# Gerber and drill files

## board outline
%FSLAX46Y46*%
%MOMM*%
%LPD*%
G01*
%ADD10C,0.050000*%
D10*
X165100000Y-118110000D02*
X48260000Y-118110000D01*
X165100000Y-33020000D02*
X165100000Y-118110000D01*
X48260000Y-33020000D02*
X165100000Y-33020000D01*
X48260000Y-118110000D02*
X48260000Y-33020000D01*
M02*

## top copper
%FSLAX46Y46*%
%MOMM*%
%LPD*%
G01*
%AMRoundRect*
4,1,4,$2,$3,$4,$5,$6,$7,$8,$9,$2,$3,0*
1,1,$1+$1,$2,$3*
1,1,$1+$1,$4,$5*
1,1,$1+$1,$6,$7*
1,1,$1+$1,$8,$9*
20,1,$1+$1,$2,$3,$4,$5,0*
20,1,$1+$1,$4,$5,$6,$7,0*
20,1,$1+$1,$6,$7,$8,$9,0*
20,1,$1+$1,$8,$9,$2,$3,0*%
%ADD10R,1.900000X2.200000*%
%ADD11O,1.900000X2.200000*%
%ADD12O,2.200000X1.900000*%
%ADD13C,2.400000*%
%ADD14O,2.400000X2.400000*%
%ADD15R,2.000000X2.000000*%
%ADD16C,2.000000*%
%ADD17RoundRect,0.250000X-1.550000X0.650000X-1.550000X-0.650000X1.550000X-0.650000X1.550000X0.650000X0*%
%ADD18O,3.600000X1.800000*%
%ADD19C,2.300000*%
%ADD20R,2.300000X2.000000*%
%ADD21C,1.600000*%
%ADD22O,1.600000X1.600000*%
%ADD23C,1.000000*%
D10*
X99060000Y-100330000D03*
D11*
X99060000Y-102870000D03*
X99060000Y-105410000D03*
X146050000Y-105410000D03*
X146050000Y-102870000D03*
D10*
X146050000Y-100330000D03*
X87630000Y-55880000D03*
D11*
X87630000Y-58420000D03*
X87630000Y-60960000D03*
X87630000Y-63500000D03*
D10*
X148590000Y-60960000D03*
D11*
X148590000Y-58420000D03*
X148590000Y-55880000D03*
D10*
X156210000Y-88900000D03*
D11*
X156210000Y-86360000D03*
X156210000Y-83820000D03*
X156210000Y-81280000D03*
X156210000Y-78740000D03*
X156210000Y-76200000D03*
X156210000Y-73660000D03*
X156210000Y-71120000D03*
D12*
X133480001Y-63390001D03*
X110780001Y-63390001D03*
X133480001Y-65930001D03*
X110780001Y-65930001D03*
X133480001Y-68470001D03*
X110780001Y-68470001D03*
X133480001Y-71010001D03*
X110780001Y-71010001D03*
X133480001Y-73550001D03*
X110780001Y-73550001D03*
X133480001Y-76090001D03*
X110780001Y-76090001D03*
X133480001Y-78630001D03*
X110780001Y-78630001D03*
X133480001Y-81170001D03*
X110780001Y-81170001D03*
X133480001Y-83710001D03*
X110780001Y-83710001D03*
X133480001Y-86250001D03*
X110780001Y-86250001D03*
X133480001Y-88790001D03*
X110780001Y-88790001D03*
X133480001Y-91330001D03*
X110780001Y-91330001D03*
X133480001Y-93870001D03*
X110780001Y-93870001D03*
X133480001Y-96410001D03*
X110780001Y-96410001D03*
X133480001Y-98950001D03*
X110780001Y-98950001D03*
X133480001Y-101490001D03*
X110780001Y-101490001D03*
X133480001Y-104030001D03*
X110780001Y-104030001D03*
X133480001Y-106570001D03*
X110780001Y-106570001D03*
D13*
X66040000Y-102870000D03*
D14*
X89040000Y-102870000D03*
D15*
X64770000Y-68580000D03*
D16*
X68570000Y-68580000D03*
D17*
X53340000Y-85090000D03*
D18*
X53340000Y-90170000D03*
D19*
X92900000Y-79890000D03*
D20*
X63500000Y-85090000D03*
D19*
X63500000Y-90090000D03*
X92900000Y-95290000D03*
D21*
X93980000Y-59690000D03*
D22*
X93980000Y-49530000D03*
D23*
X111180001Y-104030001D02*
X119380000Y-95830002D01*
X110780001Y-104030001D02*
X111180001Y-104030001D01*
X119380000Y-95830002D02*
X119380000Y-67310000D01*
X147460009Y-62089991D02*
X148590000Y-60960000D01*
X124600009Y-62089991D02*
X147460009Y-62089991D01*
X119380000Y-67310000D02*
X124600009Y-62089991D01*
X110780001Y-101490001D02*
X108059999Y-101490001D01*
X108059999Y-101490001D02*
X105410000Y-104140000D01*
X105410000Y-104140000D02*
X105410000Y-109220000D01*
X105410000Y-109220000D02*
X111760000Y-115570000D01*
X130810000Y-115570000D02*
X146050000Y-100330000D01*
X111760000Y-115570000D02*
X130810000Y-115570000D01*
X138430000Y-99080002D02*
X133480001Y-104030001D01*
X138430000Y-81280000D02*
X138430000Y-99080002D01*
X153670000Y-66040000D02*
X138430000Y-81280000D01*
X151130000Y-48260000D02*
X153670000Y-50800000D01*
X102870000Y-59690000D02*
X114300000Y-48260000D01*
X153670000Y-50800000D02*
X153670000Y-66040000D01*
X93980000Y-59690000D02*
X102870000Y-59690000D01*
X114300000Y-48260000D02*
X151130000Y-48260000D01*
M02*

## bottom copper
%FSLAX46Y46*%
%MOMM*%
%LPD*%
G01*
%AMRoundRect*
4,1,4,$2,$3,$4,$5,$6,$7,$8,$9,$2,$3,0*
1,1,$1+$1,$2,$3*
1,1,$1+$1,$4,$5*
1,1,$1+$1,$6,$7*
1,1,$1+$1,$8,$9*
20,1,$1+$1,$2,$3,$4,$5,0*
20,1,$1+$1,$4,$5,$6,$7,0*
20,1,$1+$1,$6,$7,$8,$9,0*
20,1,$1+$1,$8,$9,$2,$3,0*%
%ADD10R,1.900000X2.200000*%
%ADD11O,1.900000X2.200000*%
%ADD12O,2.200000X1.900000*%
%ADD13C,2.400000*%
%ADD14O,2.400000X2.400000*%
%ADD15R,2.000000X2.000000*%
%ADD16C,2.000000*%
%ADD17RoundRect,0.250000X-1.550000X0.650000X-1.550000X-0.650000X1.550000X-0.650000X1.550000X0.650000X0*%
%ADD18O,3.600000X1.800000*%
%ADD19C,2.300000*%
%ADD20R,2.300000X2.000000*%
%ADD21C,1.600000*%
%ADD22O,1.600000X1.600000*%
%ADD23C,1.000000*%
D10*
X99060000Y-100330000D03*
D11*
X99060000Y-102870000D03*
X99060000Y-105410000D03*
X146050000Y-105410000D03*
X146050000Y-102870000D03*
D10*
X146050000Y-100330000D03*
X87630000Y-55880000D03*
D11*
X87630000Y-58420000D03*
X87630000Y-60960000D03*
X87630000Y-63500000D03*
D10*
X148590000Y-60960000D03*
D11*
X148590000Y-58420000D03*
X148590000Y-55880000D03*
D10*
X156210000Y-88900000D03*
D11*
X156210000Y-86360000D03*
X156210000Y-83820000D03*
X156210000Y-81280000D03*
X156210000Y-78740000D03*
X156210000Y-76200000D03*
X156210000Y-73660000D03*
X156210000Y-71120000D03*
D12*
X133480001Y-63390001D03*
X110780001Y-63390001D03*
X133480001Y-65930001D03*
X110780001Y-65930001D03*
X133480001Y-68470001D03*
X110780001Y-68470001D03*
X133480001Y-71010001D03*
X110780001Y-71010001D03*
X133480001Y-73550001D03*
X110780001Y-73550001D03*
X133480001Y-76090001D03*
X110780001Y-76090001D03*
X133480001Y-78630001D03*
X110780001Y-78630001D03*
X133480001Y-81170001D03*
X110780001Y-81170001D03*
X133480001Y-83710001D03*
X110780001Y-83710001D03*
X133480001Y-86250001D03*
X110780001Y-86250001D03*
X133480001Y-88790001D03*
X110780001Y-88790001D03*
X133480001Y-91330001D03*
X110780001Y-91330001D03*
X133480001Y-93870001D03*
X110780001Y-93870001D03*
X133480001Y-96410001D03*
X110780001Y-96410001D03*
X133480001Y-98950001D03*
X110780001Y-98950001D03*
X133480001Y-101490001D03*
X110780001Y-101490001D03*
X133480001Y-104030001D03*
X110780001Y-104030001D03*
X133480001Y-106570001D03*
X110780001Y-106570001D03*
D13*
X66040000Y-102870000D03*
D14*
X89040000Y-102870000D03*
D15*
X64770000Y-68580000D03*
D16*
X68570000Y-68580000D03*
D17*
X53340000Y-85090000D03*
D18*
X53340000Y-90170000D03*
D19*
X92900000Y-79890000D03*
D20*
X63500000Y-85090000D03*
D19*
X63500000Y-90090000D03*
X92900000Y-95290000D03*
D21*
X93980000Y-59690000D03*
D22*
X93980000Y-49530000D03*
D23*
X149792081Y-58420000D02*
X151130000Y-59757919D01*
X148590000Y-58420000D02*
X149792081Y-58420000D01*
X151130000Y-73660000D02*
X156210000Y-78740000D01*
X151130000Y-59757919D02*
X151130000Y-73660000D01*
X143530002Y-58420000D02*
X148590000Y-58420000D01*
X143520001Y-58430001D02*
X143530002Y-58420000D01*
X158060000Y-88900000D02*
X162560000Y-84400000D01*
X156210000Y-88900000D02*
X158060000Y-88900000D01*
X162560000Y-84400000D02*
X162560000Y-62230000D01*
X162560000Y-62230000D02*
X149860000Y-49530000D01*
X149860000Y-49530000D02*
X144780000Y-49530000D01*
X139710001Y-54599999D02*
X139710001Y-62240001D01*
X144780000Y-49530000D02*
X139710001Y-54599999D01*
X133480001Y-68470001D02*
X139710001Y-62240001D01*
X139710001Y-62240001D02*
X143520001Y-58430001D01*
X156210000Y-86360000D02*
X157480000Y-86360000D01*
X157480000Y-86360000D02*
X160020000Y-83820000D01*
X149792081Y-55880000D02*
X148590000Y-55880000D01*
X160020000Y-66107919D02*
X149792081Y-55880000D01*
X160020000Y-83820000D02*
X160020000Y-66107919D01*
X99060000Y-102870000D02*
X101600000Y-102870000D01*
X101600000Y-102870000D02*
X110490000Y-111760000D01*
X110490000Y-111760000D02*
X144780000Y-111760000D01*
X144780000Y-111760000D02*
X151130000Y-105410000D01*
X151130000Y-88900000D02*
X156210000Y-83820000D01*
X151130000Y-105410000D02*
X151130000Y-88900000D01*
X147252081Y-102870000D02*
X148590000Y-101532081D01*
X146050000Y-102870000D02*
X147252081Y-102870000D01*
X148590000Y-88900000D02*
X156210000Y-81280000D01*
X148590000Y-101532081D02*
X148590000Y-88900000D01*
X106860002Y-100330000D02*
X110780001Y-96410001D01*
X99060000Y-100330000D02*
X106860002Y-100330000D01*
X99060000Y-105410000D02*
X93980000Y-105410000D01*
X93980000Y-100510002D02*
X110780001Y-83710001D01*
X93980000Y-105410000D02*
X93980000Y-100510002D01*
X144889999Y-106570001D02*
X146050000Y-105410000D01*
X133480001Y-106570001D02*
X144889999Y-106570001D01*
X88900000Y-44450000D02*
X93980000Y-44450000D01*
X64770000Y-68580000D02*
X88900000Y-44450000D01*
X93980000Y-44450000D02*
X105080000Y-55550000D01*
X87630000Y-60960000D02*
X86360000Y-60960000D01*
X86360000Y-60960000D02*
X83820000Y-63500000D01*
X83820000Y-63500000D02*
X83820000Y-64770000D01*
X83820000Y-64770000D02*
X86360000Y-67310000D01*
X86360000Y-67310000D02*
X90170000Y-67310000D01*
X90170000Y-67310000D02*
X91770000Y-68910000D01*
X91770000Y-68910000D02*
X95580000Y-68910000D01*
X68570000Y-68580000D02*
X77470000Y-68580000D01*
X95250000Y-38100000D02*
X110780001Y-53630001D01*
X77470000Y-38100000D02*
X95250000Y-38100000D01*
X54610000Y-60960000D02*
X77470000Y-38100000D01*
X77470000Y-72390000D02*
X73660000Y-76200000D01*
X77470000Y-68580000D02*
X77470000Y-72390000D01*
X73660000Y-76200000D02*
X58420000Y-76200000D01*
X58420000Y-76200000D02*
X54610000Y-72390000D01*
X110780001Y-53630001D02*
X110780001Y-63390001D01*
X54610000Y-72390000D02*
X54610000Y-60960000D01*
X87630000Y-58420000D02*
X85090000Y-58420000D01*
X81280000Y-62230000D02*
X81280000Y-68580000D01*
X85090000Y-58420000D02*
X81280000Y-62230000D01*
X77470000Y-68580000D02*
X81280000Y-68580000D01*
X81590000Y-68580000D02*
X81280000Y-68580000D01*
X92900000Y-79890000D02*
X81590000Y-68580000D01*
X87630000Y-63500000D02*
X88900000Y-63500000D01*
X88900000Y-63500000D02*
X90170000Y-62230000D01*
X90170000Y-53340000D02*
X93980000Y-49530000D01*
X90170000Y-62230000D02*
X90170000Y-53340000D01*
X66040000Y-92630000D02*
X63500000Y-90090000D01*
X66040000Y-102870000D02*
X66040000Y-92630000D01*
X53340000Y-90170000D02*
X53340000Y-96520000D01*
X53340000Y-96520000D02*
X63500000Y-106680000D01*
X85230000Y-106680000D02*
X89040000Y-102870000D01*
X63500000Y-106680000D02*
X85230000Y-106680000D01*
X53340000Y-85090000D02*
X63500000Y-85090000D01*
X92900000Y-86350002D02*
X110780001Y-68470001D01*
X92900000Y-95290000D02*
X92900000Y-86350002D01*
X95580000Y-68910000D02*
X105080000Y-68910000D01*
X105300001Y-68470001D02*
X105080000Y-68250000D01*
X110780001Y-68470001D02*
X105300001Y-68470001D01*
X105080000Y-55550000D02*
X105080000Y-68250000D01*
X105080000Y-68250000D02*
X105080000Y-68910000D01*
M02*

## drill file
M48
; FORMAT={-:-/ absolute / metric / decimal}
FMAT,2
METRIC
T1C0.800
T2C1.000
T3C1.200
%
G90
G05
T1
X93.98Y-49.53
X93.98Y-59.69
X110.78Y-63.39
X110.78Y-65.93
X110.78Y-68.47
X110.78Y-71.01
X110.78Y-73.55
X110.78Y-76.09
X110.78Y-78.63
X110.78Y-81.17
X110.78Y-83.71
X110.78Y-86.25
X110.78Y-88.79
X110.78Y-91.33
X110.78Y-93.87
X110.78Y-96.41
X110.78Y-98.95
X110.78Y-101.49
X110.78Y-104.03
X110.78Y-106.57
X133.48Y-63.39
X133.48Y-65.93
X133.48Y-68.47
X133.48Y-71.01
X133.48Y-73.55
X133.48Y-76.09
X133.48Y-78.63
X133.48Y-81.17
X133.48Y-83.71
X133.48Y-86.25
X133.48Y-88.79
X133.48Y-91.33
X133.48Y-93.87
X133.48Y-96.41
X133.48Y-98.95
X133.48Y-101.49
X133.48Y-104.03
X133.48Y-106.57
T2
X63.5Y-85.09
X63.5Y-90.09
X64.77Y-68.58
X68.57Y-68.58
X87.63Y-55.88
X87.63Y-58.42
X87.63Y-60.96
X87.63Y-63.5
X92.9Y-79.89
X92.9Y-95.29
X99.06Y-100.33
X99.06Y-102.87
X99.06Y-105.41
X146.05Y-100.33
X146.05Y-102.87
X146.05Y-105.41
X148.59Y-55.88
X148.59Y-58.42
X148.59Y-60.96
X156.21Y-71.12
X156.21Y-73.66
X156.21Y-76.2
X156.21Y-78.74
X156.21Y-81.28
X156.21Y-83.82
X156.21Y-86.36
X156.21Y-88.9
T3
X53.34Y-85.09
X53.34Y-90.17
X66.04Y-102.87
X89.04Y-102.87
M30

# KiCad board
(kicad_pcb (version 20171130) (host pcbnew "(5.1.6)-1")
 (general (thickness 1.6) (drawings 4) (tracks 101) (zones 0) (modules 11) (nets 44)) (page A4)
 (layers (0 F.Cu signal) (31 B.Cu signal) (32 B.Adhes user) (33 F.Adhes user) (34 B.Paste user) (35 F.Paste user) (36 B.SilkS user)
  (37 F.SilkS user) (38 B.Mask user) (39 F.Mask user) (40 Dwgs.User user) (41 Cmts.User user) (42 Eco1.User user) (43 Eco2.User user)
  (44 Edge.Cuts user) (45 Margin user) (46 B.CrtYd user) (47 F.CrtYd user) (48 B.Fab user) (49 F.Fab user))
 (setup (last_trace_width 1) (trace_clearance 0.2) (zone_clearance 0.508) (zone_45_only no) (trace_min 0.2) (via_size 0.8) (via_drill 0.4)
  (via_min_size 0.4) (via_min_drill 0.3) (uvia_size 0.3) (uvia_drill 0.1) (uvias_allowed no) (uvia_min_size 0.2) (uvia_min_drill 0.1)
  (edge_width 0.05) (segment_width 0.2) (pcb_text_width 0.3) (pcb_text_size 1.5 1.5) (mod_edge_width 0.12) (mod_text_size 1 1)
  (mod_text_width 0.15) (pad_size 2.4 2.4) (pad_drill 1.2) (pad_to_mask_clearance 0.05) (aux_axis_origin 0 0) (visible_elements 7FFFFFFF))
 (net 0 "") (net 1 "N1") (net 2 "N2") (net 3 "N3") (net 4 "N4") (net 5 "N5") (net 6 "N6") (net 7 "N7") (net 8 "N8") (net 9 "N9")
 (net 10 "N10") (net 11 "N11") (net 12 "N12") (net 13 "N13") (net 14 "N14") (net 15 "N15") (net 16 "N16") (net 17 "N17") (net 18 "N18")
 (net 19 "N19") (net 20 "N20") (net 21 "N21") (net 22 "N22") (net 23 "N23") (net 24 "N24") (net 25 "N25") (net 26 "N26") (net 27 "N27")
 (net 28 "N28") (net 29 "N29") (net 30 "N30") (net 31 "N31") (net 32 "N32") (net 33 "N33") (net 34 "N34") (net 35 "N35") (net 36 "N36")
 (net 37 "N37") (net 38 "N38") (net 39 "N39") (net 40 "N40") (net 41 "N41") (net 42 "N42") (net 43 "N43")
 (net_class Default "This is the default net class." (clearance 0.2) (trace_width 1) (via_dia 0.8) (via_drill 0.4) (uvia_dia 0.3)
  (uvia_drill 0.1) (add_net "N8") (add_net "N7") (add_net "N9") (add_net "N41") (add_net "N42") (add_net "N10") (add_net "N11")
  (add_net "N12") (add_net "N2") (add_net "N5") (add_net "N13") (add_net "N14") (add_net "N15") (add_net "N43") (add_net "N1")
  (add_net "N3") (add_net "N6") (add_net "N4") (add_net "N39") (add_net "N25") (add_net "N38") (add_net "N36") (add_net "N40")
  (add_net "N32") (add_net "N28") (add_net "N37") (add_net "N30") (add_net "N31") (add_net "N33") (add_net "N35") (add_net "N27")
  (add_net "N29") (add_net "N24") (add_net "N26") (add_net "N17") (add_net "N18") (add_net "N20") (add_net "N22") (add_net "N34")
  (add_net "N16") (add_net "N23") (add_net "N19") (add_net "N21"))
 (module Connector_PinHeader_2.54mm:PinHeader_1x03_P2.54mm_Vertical (layer F.Cu) (at 99.06 100.33)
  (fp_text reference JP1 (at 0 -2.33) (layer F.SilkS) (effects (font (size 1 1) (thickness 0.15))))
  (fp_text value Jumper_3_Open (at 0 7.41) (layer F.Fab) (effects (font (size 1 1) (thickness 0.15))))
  (pad 1 thru_hole rect (at 0 0) (size 1.9 2.2) (drill 1) (layers *.Cu *.Mask) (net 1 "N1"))
  (pad 2 thru_hole oval (at 0 2.54) (size 1.9 2.2) (drill 1) (layers *.Cu *.Mask) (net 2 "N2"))
  (pad 3 thru_hole oval (at 0 5.08) (size 1.9 2.2) (drill 1) (layers *.Cu *.Mask) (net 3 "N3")))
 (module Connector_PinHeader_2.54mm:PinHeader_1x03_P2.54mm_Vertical (layer F.Cu) (at 146.05 100.33)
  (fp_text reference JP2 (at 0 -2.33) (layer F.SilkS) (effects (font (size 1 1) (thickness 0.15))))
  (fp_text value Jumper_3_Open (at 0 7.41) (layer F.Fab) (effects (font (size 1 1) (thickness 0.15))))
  (pad 3 thru_hole oval (at 0 5.08) (size 1.9 2.2) (drill 1) (layers *.Cu *.Mask) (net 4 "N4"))
  (pad 2 thru_hole oval (at 0 2.54) (size 1.9 2.2) (drill 1) (layers *.Cu *.Mask) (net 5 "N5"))
  (pad 1 thru_hole rect (at 0 0) (size 1.9 2.2) (drill 1) (layers *.Cu *.Mask) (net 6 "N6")))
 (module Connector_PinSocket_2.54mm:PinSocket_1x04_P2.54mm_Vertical (layer F.Cu) (at 87.63 55.88)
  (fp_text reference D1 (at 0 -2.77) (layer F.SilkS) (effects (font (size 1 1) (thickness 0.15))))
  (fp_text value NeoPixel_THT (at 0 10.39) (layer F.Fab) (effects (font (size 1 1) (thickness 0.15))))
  (pad 1 thru_hole rect (at 0 0) (size 1.9 2.2) (drill 1) (layers *.Cu *.Mask) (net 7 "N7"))
  (pad 2 thru_hole oval (at 0 2.54) (size 1.9 2.2) (drill 1) (layers *.Cu *.Mask) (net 7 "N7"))
  (pad 3 thru_hole oval (at 0 5.08) (size 1.9 2.2) (drill 1) (layers *.Cu *.Mask) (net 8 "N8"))
  (pad 4 thru_hole oval (at 0 7.62) (size 1.9 2.2) (drill 1) (layers *.Cu *.Mask) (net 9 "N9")))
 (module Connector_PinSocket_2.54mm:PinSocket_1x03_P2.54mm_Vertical (layer F.Cu) (at 148.59 60.96 180)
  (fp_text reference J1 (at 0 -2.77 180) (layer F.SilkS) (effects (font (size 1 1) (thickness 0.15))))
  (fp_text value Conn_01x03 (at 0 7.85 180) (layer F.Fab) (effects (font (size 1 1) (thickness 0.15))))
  (pad 1 thru_hole rect (at 0 0 180) (size 1.9 2.2) (drill 1) (layers *.Cu *.Mask) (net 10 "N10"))
  (pad 2 thru_hole oval (at 0 2.54 180) (size 1.9 2.2) (drill 1) (layers *.Cu *.Mask) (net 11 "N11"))
  (pad 3 thru_hole oval (at 0 5.08 180) (size 1.9 2.2) (drill 1) (layers *.Cu *.Mask) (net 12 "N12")))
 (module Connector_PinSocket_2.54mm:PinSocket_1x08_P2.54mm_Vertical (layer F.Cu) (at 156.21 88.9 180)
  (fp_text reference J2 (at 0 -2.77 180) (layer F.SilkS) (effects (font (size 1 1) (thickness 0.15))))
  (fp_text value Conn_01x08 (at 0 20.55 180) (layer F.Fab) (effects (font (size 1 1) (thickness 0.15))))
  (pad 1 thru_hole rect (at 0 0 180) (size 1.9 2.2) (drill 1) (layers *.Cu *.Mask) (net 11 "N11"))
  (pad 2 thru_hole oval (at 0 2.54 180) (size 1.9 2.2) (drill 1) (layers *.Cu *.Mask) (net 12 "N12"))
  (pad 3 thru_hole oval (at 0 5.08 180) (size 1.9 2.2) (drill 1) (layers *.Cu *.Mask) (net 2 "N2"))
  (pad 4 thru_hole oval (at 0 7.62 180) (size 1.9 2.2) (drill 1) (layers *.Cu *.Mask) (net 5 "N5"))
  (pad 5 thru_hole oval (at 0 10.16 180) (size 1.9 2.2) (drill 1) (layers *.Cu *.Mask) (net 11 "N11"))
  (pad 6 thru_hole oval (at 0 12.7 180) (size 1.9 2.2) (drill 1) (layers *.Cu *.Mask) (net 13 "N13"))
  (pad 7 thru_hole oval (at 0 15.24 180) (size 1.9 2.2) (drill 1) (layers *.Cu *.Mask) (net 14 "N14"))
  (pad 8 thru_hole oval (at 0 17.78 180) (size 1.9 2.2) (drill 1) (layers *.Cu *.Mask) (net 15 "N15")))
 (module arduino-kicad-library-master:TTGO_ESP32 (layer F.Cu) (at 122.130001 86.250001)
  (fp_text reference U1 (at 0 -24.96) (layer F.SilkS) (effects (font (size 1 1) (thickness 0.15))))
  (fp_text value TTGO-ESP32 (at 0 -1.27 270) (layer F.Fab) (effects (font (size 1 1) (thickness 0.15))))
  (pad GND thru_hole oval (at 11.35 -22.86 270) (size 1.9 2.2) (drill 0.8) (layers *.Cu *.Mask) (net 7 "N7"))
  (pad GND thru_hole oval (at -11.35 -22.86 270) (size 1.9 2.2) (drill 0.8) (layers *.Cu *.Mask) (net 7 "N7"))
  (pad 5V thru_hole oval (at 11.35 -20.32 270) (size 1.9 2.2) (drill 0.8) (layers *.Cu *.Mask) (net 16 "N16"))
  (pad 5V thru_hole oval (at -11.35 -20.32 270) (size 1.9 2.2) (drill 0.8) (layers *.Cu *.Mask) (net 16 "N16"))
  (pad 3V3 thru_hole oval (at 11.35 -17.78 270) (size 1.9 2.2) (drill 0.8) (layers *.Cu *.Mask) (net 8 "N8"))
  (pad 3V3 thru_hole oval (at -11.35 -17.78 270) (size 1.9 2.2) (drill 0.8) (layers *.Cu *.Mask) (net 8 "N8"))
  (pad 36 thru_hole oval (at 11.35 -15.24 270) (size 1.9 2.2) (drill 0.8) (layers *.Cu *.Mask) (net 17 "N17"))
  (pad GND thru_hole oval (at -11.35 -15.24 270) (size 1.9 2.2) (drill 0.8) (layers *.Cu *.Mask) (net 7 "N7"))
  (pad 37 thru_hole oval (at 11.35 -12.7 270) (size 1.9 2.2) (drill 0.8) (layers *.Cu *.Mask) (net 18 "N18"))
  (pad RX thru_hole oval (at -11.35 -12.7 270) (size 1.9 2.2) (drill 0.8) (layers *.Cu *.Mask) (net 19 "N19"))
  (pad 38 thru_hole oval (at 11.35 -10.16 270) (size 1.9 2.2) (drill 0.8) (layers *.Cu *.Mask) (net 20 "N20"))
  (pad TX thru_hole oval (at -11.35 -10.16 270) (size 1.9 2.2) (drill 0.8) (layers *.Cu *.Mask) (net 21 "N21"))
  (pad 39 thru_hole oval (at 11.35 -7.62 270) (size 1.9 2.2) (drill 0.8) (layers *.Cu *.Mask) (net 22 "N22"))
  (pad RST thru_hole oval (at -11.35 -7.62 270) (size 1.9 2.2) (drill 0.8) (layers *.Cu *.Mask) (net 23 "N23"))
  (pad 34 thru_hole oval (at 11.35 -5.08 270) (size 1.9 2.2) (drill 0.8) (layers *.Cu *.Mask) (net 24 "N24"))
  (pad 0 thru_hole oval (at -11.35 -5.08 270) (size 1.9 2.2) (drill 0.8) (layers *.Cu *.Mask) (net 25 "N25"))
  (pad 35 thru_hole oval (at 11.35 -2.54 270) (size 1.9 2.2) (drill 0.8) (layers *.Cu *.Mask) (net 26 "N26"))
  (pad 22 thru_hole oval (at -11.35 -2.54 270) (size 1.9 2.2) (drill 0.8) (layers *.Cu *.Mask) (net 3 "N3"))
  (pad 32 thru_hole oval (at 11.35 0 270) (size 1.9 2.2) (drill 0.8) (layers *.Cu *.Mask) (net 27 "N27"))
  (pad 19 thru_hole oval (at -11.35 0 270) (size 1.9 2.2) (drill 0.8) (layers *.Cu *.Mask) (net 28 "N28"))
  (pad 33 thru_hole oval (at 11.35 2.54 270) (size 1.9 2.2) (drill 0.8) (layers *.Cu *.Mask) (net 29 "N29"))
  (pad 23 thru_hole oval (at -11.35 2.54 270) (size 1.9 2.2) (drill 0.8) (layers *.Cu *.Mask) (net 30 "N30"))
  (pad 25 thru_hole oval (at 11.35 5.08 270) (size 1.9 2.2) (drill 0.8) (layers *.Cu *.Mask) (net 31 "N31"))
  (pad 18 thru_hole oval (at -11.35 5.08 270) (size 1.9 2.2) (drill 0.8) (layers *.Cu *.Mask) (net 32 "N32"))
  (pad 26 thru_hole oval (at 11.35 7.62 270) (size 1.9 2.2) (drill 0.8) (layers *.Cu *.Mask) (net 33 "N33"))
  (pad 5 thru_hole oval (at -11.35 7.62 270) (size 1.9 2.2) (drill 0.8) (layers *.Cu *.Mask) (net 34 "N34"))
  (pad 27 thru_hole oval (at 11.35 10.16 270) (size 1.9 2.2) (drill 0.8) (layers *.Cu *.Mask) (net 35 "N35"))
  (pad 15 thru_hole oval (at -11.35 10.16 270) (size 1.9 2.2) (drill 0.8) (layers *.Cu *.Mask) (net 1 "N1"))
  (pad 14 thru_hole oval (at 11.35 12.7 270) (size 1.9 2.2) (drill 0.8) (layers *.Cu *.Mask) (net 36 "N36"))
  (pad 2 thru_hole oval (at -11.35 12.7 270) (size 1.9 2.2) (drill 0.8) (layers *.Cu *.Mask) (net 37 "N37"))
  (pad 12 thru_hole oval (at 11.35 15.24 270) (size 1.9 2.2) (drill 0.8) (layers *.Cu *.Mask) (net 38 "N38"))
  (pad 4 thru_hole oval (at -11.35 15.24 270) (size 1.9 2.2) (drill 0.8) (layers *.Cu *.Mask) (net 6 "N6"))
  (pad 13 thru_hole oval (at 11.35 17.78 270) (size 1.9 2.2) (drill 0.8) (layers *.Cu *.Mask) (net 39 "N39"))
  (pad 17 thru_hole oval (at -11.35 17.78 270) (size 1.9 2.2) (drill 0.8) (layers *.Cu *.Mask) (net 10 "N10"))
  (pad 21 thru_hole oval (at 11.35 20.32 270) (size 1.9 2.2) (drill 0.8) (layers *.Cu *.Mask) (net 4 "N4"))
  (pad 16 thru_hole oval (at -11.35 20.32 270) (size 1.9 2.2) (drill 0.8) (layers *.Cu *.Mask) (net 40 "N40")))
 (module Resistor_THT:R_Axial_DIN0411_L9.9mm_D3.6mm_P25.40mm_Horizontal (layer F.Cu) (at 66.04 102.87)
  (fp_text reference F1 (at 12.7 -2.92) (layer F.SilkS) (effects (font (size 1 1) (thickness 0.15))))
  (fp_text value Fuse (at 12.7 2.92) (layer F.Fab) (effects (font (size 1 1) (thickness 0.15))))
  (pad 1 thru_hole circle (at 0 0) (size 2.4 2.4) (drill 1.2) (layers *.Cu *.Mask) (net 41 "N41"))
  (pad 2 thru_hole oval (at 23 0) (size 2.4 2.4) (drill 1.2) (layers *.Cu *.Mask) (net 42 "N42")))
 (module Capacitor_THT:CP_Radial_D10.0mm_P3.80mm (layer F.Cu) (at 64.77 68.58)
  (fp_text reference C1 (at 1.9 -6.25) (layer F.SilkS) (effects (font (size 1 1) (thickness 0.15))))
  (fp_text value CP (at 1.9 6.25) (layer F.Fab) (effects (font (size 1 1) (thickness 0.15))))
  (pad 1 thru_hole rect (at 0 0) (size 2 2) (drill 1) (layers *.Cu *.Mask) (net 8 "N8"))
  (pad 2 thru_hole circle (at 3.8 0) (size 2 2) (drill 1) (layers *.Cu *.Mask) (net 7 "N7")))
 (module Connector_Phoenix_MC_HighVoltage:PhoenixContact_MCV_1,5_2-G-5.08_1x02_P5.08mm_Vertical (layer F.Cu) (at 53.34 85.09 270)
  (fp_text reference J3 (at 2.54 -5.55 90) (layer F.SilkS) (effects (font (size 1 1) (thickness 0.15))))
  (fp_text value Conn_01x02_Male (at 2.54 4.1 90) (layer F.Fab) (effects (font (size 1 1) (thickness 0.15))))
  (pad 1 thru_hole roundrect (at 0 0 270) (size 1.8 3.6) (drill 1.2) (layers *.Cu *.Mask) (roundrect_rratio 0.138889) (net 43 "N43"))
  (pad 2 thru_hole oval (at 5.08 0 270) (size 1.8 3.6) (drill 1.2) (layers *.Cu *.Mask) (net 42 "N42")))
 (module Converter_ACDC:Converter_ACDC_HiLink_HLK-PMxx (layer F.Cu) (at 63.5 85.09)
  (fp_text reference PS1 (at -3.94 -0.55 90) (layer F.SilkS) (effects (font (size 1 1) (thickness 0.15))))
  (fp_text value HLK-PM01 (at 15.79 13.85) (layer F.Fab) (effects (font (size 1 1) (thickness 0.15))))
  (pad 3 thru_hole circle (at 29.4 -5.2) (size 2.3 2.3) (drill 1) (layers *.Cu *.Mask) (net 7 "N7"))
  (pad 1 thru_hole rect (at 0 0) (size 2.3 2) (drill 1) (layers *.Cu *.Mask) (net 43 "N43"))
  (pad 2 thru_hole circle (at 0 5) (size 2.3 2.3) (drill 1) (layers *.Cu *.Mask) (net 41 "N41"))
  (pad 4 thru_hole circle (at 29.4 10.2) (size 2.3 2.3) (drill 1) (layers *.Cu *.Mask) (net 8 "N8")))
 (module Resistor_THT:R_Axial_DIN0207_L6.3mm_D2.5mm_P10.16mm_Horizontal (layer F.Cu) (at 93.98 59.69 90)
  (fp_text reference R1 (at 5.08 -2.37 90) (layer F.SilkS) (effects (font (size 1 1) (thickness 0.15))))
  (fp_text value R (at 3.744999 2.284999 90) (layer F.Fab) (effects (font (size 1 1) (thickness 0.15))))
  (pad 1 thru_hole circle (at 0 0 90) (size 1.6 1.6) (drill 0.8) (layers *.Cu *.Mask) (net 39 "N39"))
  (pad 2 thru_hole oval (at 10.16 0 90) (size 1.6 1.6) (drill 0.8) (layers *.Cu *.Mask) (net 9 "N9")))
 (gr_line (start 165.1 118.11) (end 48.26 118.11) (layer Edge.Cuts) (width 0.05))
 (gr_line (start 165.1 33.02) (end 165.1 118.11) (layer Edge.Cuts) (width 0.05))
 (gr_line (start 48.26 33.02) (end 165.1 33.02) (layer Edge.Cuts) (width 0.05))
 (gr_line (start 48.26 118.11) (end 48.26 33.02) (layer Edge.Cuts) (width 0.05))
 (segment (start 111.180001 104.030001) (end 119.38 95.830002) (width 1) (layer F.Cu) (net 10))
 (segment (start 110.780001 104.030001) (end 111.180001 104.030001) (width 1) (layer F.Cu) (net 10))
 (segment (start 119.38 95.830002) (end 119.38 67.31) (width 1) (layer F.Cu) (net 10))
 (segment (start 147.460009 62.089991) (end 148.59 60.96) (width 1) (layer F.Cu) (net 10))
 (segment (start 124.600009 62.089991) (end 147.460009 62.089991) (width 1) (layer F.Cu) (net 10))
 (segment (start 119.38 67.31) (end 124.600009 62.089991) (width 1) (layer F.Cu) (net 10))
 (segment (start 149.792081 58.42) (end 151.13 59.757919) (width 1) (layer B.Cu) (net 11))
 (segment (start 148.59 58.42) (end 149.792081 58.42) (width 1) (layer B.Cu) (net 11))
 (segment (start 151.13 73.66) (end 156.21 78.74) (width 1) (layer B.Cu) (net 11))
 (segment (start 151.13 59.757919) (end 151.13 73.66) (width 1) (layer B.Cu) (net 11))
 (segment (start 143.530002 58.42) (end 148.59 58.42) (width 1) (layer B.Cu) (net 11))
 (segment (start 143.520001 58.430001) (end 143.530002 58.42) (width 1) (layer B.Cu) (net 11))
 (segment (start 158.06 88.9) (end 162.56 84.4) (width 1) (layer B.Cu) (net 11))
 (segment (start 156.21 88.9) (end 158.06 88.9) (width 1) (layer B.Cu) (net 11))
 (segment (start 162.56 84.4) (end 162.56 62.23) (width 1) (layer B.Cu) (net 11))
 (segment (start 162.56 62.23) (end 149.86 49.53) (width 1) (layer B.Cu) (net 11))
 (segment (start 149.86 49.53) (end 144.78 49.53) (width 1) (layer B.Cu) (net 11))
 (segment (start 139.710001 54.599999) (end 139.710001 62.240001) (width 1) (layer B.Cu) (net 11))
 (segment (start 144.78 49.53) (end 139.710001 54.599999) (width 1) (layer B.Cu) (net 11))
 (segment (start 133.480001 68.470001) (end 139.710001 62.240001) (width 1) (layer B.Cu) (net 11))
 (segment (start 139.710001 62.240001) (end 143.520001 58.430001) (width 1) (layer B.Cu) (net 11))
 (segment (start 156.21 86.36) (end 157.48 86.36) (width 1) (layer B.Cu) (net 12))
 (segment (start 157.48 86.36) (end 160.02 83.82) (width 1) (layer B.Cu) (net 12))
 (segment (start 149.792081 55.88) (end 148.59 55.88) (width 1) (layer B.Cu) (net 12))
 (segment (start 160.02 66.107919) (end 149.792081 55.88) (width 1) (layer B.Cu) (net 12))
 (segment (start 160.02 83.82) (end 160.02 66.107919) (width 1) (layer B.Cu) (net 12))
 (segment (start 99.06 102.87) (end 101.6 102.87) (width 1) (layer B.Cu) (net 2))
 (segment (start 101.6 102.87) (end 110.49 111.76) (width 1) (layer B.Cu) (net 2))
 (segment (start 110.49 111.76) (end 144.78 111.76) (width 1) (layer B.Cu) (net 2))
 (segment (start 144.78 111.76) (end 151.13 105.41) (width 1) (layer B.Cu) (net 2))
 (segment (start 151.13 88.9) (end 156.21 83.82) (width 1) (layer B.Cu) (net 2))
 (segment (start 151.13 105.41) (end 151.13 88.9) (width 1) (layer B.Cu) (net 2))
 (segment (start 147.252081 102.87) (end 148.59 101.532081) (width 1) (layer B.Cu) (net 5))
 (segment (start 146.05 102.87) (end 147.252081 102.87) (width 1) (layer B.Cu) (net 5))
 (segment (start 148.59 88.9) (end 156.21 81.28) (width 1) (layer B.Cu) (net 5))
 (segment (start 148.59 101.532081) (end 148.59 88.9) (width 1) (layer B.Cu) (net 5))
 (segment (start 106.860002 100.33) (end 110.780001 96.410001) (width 1) (layer B.Cu) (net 1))
 (segment (start 99.06 100.33) (end 106.860002 100.33) (width 1) (layer B.Cu) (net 1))
 (segment (start 99.06 105.41) (end 93.98 105.41) (width 1) (layer B.Cu) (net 3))
 (segment (start 93.98 100.510002) (end 110.780001 83.710001) (width 1) (layer B.Cu) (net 3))
 (segment (start 93.98 105.41) (end 93.98 100.510002) (width 1) (layer B.Cu) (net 3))
 (segment (start 144.889999 106.570001) (end 146.05 105.41) (width 1) (layer B.Cu) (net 4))
 (segment (start 133.480001 106.570001) (end 144.889999 106.570001) (width 1) (layer B.Cu) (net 4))
 (segment (start 110.780001 101.490001) (end 108.059999 101.490001) (width 1) (layer F.Cu) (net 6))
 (segment (start 108.059999 101.490001) (end 105.41 104.14) (width 1) (layer F.Cu) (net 6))
 (segment (start 105.41 104.14) (end 105.41 109.22) (width 1) (layer F.Cu) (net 6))
 (segment (start 105.41 109.22) (end 111.76 115.57) (width 1) (layer F.Cu) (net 6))
 (segment (start 130.81 115.57) (end 146.05 100.33) (width 1) (layer F.Cu) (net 6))
 (segment (start 111.76 115.57) (end 130.81 115.57) (width 1) (layer F.Cu) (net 6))
 (segment (start 88.9 44.45) (end 93.98 44.45) (width 1) (layer B.Cu) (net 8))
 (segment (start 64.77 68.58) (end 88.9 44.45) (width 1) (layer B.Cu) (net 8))
 (segment (start 93.98 44.45) (end 105.08 55.55) (width 1) (layer B.Cu) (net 8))
 (segment (start 87.63 60.96) (end 86.36 60.96) (width 1) (layer B.Cu) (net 8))
 (segment (start 86.36 60.96) (end 83.82 63.5) (width 1) (layer B.Cu) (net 8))
 (segment (start 83.82 63.5) (end 83.82 64.77) (width 1) (layer B.Cu) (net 8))
 (segment (start 83.82 64.77) (end 86.36 67.31) (width 1) (layer B.Cu) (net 8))
 (segment (start 86.36 67.31) (end 90.17 67.31) (width 1) (layer B.Cu) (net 8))
 (segment (start 90.17 67.31) (end 91.77 68.91) (width 1) (layer B.Cu) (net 8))
 (segment (start 91.77 68.91) (end 95.58 68.91) (width 1) (layer B.Cu) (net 8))
 (segment (start 68.57 68.58) (end 77.47 68.58) (width 1) (layer B.Cu) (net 7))
 (segment (start 95.25 38.1) (end 110.780001 53.630001) (width 1) (layer B.Cu) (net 7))
 (segment (start 77.47 38.1) (end 95.25 38.1) (width 1) (layer B.Cu) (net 7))
 (segment (start 54.61 60.96) (end 77.47 38.1) (width 1) (layer B.Cu) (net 7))
 (segment (start 77.47 72.39) (end 73.66 76.2) (width 1) (layer B.Cu) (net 7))
 (segment (start 77.47 68.58) (end 77.47 72.39) (width 1) (layer B.Cu) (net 7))
 (segment (start 73.66 76.2) (end 58.42 76.2) (width 1) (layer B.Cu) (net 7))
 (segment (start 58.42 76.2) (end 54.61 72.39) (width 1) (layer B.Cu) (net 7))
 (segment (start 110.780001 53.630001) (end 110.780001 63.390001) (width 1) (layer B.Cu) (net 7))
 (segment (start 54.61 72.39) (end 54.61 60.96) (width 1) (layer B.Cu) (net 7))
 (segment (start 87.63 58.42) (end 85.09 58.42) (width 1) (layer B.Cu) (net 7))
 (segment (start 81.28 62.23) (end 81.28 68.58) (width 1) (layer B.Cu) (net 7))
 (segment (start 85.09 58.42) (end 81.28 62.23) (width 1) (layer B.Cu) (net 7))
 (segment (start 77.47 68.58) (end 81.28 68.58) (width 1) (layer B.Cu) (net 7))
 (segment (start 81.59 68.58) (end 81.28 68.58) (width 1) (layer B.Cu) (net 7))
 (segment (start 92.9 79.89) (end 81.59 68.58) (width 1) (layer B.Cu) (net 7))
 (segment (start 87.63 63.5) (end 88.9 63.5) (width 1) (layer B.Cu) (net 9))
 (segment (start 88.9 63.5) (end 90.17 62.23) (width 1) (layer B.Cu) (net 9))
 (segment (start 90.17 53.34) (end 93.98 49.53) (width 1) (layer B.Cu) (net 9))
 (segment (start 90.17 62.23) (end 90.17 53.34) (width 1) (layer B.Cu) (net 9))
 (segment (start 66.04 92.63) (end 63.5 90.09) (width 1) (layer B.Cu) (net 41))
 (segment (start 66.04 102.87) (end 66.04 92.63) (width 1) (layer B.Cu) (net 41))
 (segment (start 53.34 90.17) (end 53.34 96.52) (width 1) (layer B.Cu) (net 42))
 (segment (start 53.34 96.52) (end 63.5 106.68) (width 1) (layer B.Cu) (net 42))
 (segment (start 85.23 106.68) (end 89.04 102.87) (width 1) (layer B.Cu) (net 42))
 (segment (start 63.5 106.68) (end 85.23 106.68) (width 1) (layer B.Cu) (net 42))
 (segment (start 53.34 85.09) (end 63.5 85.09) (width 1) (layer B.Cu) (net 43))
 (segment (start 92.9 86.350002) (end 110.780001 68.470001) (width 1) (layer B.Cu) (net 8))
 (segment (start 92.9 95.29) (end 92.9 86.350002) (width 1) (layer B.Cu) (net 8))
 (segment (start 95.58 68.91) (end 105.08 68.91) (width 1) (layer B.Cu) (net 8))
 (segment (start 105.300001 68.470001) (end 105.08 68.25) (width 1) (layer B.Cu) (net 8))
 (segment (start 110.780001 68.470001) (end 105.300001 68.470001) (width 1) (layer B.Cu) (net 8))
 (segment (start 105.08 55.55) (end 105.08 68.25) (width 1) (layer B.Cu) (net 8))
 (segment (start 105.08 68.25) (end 105.08 68.91) (width 1) (layer B.Cu) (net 8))
 (segment (start 138.43 99.080002) (end 133.480001 104.030001) (width 1) (layer F.Cu) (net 39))
 (segment (start 138.43 81.28) (end 138.43 99.080002) (width 1) (layer F.Cu) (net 39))
 (segment (start 153.67 66.04) (end 138.43 81.28) (width 1) (layer F.Cu) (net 39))
 (segment (start 151.13 48.26) (end 153.67 50.8) (width 1) (layer F.Cu) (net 39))
 (segment (start 102.87 59.69) (end 114.3 48.26) (width 1) (layer F.Cu) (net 39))
 (segment (start 153.67 50.8) (end 153.67 66.04) (width 1) (layer F.Cu) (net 39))
 (segment (start 93.98 59.69) (end 102.87 59.69) (width 1) (layer F.Cu) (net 39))
 (segment (start 114.3 48.26) (end 151.13 48.26) (width 1) (layer F.Cu) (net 39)))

